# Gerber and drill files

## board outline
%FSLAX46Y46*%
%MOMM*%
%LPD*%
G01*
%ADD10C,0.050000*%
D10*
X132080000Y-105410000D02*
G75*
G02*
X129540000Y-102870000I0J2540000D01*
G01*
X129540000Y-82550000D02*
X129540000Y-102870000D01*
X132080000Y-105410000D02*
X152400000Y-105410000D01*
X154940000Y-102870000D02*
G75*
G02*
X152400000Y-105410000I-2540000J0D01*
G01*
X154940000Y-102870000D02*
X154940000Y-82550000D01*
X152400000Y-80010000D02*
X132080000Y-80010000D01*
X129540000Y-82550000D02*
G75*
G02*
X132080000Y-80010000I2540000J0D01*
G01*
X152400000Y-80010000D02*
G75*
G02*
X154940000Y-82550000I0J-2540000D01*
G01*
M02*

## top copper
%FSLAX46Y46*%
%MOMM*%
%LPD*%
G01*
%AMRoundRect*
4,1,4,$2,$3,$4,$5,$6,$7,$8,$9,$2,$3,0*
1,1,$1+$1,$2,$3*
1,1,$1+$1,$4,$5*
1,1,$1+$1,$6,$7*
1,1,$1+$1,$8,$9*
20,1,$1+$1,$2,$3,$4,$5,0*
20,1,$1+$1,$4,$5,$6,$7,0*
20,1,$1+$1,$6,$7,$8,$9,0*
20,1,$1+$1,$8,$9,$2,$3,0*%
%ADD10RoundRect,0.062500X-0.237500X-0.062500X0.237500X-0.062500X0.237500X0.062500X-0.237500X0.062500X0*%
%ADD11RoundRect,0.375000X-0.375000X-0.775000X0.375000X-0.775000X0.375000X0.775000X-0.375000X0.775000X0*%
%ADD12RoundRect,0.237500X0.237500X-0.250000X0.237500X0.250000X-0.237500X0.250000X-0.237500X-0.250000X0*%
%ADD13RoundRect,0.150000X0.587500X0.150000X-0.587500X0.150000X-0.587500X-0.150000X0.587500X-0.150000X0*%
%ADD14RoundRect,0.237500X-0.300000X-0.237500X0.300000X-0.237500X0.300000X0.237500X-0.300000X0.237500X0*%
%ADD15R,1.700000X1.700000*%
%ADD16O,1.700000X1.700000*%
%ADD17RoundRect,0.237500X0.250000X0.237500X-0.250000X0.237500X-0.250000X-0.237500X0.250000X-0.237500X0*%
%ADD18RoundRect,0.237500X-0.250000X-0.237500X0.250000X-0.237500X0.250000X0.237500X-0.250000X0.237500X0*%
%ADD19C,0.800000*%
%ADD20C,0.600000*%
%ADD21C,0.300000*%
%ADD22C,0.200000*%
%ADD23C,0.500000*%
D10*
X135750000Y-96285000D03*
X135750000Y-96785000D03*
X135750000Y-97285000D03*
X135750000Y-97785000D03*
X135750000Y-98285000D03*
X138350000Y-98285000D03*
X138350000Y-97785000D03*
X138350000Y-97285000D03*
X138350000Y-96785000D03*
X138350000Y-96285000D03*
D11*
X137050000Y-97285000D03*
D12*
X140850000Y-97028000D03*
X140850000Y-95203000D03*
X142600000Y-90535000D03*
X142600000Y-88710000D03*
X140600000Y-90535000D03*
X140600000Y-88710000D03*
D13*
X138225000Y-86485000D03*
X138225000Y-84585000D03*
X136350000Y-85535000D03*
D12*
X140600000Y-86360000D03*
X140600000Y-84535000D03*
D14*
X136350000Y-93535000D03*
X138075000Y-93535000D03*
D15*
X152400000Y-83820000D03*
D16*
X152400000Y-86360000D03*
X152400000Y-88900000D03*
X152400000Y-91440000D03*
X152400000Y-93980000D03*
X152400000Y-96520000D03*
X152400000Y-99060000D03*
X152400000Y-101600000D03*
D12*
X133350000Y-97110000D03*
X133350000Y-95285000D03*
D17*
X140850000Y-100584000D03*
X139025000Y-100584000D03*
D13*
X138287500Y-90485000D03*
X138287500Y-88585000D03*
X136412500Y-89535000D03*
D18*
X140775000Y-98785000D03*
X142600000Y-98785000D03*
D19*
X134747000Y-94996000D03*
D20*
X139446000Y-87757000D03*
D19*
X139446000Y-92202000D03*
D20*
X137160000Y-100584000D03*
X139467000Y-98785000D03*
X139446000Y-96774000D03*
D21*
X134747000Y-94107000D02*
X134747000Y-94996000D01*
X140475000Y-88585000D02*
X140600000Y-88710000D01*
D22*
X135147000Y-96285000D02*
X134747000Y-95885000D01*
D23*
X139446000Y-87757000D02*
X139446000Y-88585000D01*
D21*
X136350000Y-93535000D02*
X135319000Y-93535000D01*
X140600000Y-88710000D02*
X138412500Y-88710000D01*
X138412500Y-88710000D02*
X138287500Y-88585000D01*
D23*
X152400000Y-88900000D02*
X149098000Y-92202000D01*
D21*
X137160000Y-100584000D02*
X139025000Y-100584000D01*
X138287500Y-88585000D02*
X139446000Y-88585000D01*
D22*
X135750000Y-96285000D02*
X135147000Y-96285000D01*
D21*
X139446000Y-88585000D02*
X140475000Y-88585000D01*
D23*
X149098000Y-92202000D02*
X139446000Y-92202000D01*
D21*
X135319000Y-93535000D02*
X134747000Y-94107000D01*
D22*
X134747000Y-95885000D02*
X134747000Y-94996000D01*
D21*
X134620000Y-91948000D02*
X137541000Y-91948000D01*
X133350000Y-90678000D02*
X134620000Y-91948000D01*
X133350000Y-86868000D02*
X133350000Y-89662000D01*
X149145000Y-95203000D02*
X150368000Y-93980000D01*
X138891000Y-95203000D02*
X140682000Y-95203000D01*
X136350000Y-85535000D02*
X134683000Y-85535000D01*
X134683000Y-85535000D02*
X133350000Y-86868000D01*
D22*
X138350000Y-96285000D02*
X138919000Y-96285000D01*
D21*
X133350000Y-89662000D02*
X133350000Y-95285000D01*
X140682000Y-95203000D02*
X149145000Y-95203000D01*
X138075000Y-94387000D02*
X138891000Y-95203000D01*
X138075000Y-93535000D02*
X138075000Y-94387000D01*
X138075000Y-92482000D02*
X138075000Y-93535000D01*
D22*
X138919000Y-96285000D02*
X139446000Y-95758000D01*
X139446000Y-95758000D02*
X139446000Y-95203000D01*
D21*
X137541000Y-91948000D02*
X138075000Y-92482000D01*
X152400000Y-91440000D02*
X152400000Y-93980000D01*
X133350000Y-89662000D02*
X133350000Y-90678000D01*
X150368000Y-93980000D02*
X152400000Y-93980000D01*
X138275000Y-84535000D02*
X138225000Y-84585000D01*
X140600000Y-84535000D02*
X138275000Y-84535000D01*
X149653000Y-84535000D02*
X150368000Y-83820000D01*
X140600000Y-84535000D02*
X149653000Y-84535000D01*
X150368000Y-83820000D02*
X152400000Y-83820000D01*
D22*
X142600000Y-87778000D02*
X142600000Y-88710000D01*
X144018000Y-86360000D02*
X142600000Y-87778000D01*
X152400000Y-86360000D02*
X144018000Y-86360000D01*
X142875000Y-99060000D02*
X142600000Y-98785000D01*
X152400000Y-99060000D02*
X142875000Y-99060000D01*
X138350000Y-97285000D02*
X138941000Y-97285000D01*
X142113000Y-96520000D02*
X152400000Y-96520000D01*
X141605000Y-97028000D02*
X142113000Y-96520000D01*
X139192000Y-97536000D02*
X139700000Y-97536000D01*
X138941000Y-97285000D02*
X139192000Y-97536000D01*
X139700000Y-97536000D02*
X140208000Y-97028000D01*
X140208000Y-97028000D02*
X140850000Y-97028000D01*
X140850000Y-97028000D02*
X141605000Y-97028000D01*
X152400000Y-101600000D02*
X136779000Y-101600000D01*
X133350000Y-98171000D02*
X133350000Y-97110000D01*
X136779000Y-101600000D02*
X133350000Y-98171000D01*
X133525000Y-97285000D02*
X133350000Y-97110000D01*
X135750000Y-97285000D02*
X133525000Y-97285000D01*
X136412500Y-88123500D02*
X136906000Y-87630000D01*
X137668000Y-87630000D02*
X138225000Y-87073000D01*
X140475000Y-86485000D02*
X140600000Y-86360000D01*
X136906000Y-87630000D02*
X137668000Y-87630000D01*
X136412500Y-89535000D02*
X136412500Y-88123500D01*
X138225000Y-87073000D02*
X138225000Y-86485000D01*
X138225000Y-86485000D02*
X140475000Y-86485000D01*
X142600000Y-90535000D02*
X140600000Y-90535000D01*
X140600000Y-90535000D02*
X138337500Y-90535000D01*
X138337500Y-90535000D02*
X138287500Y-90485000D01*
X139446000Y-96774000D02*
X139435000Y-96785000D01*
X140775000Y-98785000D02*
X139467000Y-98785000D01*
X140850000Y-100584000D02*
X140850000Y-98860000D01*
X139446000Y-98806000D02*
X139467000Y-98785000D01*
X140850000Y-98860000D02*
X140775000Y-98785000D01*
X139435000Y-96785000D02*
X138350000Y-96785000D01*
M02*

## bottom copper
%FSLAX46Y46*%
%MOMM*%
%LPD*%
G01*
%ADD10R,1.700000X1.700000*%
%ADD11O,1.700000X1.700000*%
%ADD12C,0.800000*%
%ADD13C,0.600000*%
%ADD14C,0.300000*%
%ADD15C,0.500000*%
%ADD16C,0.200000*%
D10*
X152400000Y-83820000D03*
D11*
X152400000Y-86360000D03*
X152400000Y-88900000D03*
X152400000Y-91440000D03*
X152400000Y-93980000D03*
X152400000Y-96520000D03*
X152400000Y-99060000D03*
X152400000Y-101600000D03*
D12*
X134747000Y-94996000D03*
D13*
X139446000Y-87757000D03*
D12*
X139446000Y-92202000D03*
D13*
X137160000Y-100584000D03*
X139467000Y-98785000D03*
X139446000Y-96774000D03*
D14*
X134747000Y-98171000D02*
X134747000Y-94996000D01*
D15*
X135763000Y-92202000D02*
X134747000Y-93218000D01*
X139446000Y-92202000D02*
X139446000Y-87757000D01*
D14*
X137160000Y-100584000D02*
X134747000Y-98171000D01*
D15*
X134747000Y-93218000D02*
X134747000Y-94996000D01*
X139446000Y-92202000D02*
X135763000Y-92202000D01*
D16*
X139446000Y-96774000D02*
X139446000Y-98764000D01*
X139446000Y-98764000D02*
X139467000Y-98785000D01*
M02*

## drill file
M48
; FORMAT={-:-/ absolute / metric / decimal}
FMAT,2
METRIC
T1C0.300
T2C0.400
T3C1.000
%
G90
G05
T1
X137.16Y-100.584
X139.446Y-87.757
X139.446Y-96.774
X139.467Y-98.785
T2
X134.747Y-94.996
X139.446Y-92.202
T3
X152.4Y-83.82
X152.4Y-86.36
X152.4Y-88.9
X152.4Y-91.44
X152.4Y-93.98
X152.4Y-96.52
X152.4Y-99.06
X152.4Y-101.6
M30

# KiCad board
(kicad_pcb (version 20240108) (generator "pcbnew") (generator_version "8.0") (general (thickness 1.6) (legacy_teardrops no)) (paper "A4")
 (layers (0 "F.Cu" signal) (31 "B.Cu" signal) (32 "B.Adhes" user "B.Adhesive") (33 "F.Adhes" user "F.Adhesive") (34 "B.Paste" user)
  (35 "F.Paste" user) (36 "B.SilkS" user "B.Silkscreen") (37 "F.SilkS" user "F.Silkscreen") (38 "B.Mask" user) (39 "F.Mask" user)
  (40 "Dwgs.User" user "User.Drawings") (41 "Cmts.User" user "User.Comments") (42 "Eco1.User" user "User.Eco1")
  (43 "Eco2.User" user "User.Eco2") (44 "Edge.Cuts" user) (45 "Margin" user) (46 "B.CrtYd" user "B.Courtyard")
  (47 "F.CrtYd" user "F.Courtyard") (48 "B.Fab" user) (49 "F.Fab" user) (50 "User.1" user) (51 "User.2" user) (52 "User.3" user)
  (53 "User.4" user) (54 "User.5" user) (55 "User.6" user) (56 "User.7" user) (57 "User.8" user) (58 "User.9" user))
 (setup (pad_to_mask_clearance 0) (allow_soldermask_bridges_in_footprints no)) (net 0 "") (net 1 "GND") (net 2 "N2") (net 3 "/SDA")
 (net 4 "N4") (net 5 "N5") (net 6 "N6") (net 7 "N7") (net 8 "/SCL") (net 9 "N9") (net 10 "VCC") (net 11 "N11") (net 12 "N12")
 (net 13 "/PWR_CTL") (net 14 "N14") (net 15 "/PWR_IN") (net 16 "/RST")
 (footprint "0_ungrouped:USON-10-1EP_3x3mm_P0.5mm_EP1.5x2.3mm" (layer "F.Cu") (at 137.05 97.285)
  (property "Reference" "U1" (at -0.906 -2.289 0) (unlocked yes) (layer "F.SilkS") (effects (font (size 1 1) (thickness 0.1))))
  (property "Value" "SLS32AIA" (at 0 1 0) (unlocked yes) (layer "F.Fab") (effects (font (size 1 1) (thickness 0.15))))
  (pad "1" smd roundrect (at -1.3 -1) (size 0.6 0.25) (layers "F.Cu" "F.Paste" "F.Mask") (roundrect_rratio 0.25) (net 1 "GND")
   (thermal_bridge_angle 45))
  (pad "2" smd roundrect (at -1.3 -0.5) (size 0.6 0.25) (layers "F.Cu" "F.Paste" "F.Mask") (roundrect_rratio 0.25) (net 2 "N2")
   (thermal_bridge_angle 45))
  (pad "3" smd roundrect (at -1.3 0) (size 0.6 0.25) (layers "F.Cu" "F.Paste" "F.Mask") (roundrect_rratio 0.25) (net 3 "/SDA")
   (thermal_bridge_angle 45))
  (pad "4" smd roundrect (at -1.3 0.5) (size 0.6 0.25) (layers "F.Cu" "F.Paste" "F.Mask") (roundrect_rratio 0.25) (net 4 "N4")
   (thermal_bridge_angle 45))
  (pad "5" smd roundrect (at -1.3 1) (size 0.6 0.25) (layers "F.Cu" "F.Paste" "F.Mask") (roundrect_rratio 0.25) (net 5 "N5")
   (thermal_bridge_angle 45))
  (pad "6" smd roundrect (at 1.3 1) (size 0.6 0.25) (layers "F.Cu" "F.Paste" "F.Mask") (roundrect_rratio 0.25) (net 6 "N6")
   (thermal_bridge_angle 45))
  (pad "7" smd roundrect (at 1.3 0.5) (size 0.6 0.25) (layers "F.Cu" "F.Paste" "F.Mask") (roundrect_rratio 0.25) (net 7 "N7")
   (thermal_bridge_angle 45))
  (pad "8" smd roundrect (at 1.3 0) (size 0.6 0.25) (layers "F.Cu" "F.Paste" "F.Mask") (roundrect_rratio 0.25) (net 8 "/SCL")
   (thermal_bridge_angle 45))
  (pad "9" smd roundrect (at 1.3 -0.5) (size 0.6 0.25) (layers "F.Cu" "F.Paste" "F.Mask") (roundrect_rratio 0.25) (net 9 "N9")
   (thermal_bridge_angle 45))
  (pad "10" smd roundrect (at 1.3 -1) (size 0.6 0.25) (layers "F.Cu" "F.Paste" "F.Mask") (roundrect_rratio 0.25) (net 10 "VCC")
   (thermal_bridge_angle 45))
  (pad "11" smd roundrect (at 0 0) (size 1.5 2.3) (layers "F.Cu" "F.Paste" "F.Mask") (roundrect_rratio 0.25) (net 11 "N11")
   (thermal_bridge_angle 45)))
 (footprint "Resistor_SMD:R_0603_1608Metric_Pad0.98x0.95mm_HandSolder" (layer "F.Cu") (at 140.85 96.1155 90)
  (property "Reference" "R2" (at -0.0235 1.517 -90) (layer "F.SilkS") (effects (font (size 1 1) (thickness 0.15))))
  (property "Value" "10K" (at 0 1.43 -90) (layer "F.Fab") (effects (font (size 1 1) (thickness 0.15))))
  (pad "1" smd roundrect (at -0.9125 0 90) (size 0.975 0.95) (layers "F.Cu" "F.Paste" "F.Mask") (roundrect_rratio 0.25) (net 8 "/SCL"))
  (pad "2" smd roundrect (at 0.9125 0 90) (size 0.975 0.95) (layers "F.Cu" "F.Paste" "F.Mask") (roundrect_rratio 0.25) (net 10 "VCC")))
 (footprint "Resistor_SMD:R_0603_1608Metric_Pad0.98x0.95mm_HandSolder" (layer "F.Cu") (at 142.6 89.6225 90)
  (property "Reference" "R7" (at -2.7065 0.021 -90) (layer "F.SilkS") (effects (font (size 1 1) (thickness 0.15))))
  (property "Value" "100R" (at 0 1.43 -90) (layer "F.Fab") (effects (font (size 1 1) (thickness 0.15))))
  (pad "1" smd roundrect (at -0.9125 0 90) (size 0.975 0.95) (layers "F.Cu" "F.Paste" "F.Mask") (roundrect_rratio 0.25) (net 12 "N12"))
  (pad "2" smd roundrect (at 0.9125 0 90) (size 0.975 0.95) (layers "F.Cu" "F.Paste" "F.Mask") (roundrect_rratio 0.25) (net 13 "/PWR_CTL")))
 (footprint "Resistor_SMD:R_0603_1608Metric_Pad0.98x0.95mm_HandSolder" (layer "F.Cu") (at 140.6 89.6225 90)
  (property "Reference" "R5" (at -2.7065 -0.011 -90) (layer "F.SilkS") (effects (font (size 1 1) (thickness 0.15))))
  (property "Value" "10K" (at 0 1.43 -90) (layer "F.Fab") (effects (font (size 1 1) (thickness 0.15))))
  (pad "1" smd roundrect (at -0.9125 0 90) (size 0.975 0.95) (layers "F.Cu" "F.Paste" "F.Mask") (roundrect_rratio 0.25) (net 12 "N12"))
  (pad "2" smd roundrect (at 0.9125 0 90) (size 0.975 0.95) (layers "F.Cu" "F.Paste" "F.Mask") (roundrect_rratio 0.25) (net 1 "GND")))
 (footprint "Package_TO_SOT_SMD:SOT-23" (layer "F.Cu") (at 137.2875 85.535 180)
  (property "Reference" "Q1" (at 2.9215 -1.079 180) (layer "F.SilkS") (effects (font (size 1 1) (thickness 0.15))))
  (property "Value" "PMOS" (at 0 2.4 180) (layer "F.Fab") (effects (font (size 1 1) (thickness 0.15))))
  (pad "1" smd roundrect (at -0.9375 -0.95 180) (size 1.475 0.6) (layers "F.Cu" "F.Paste" "F.Mask") (roundrect_rratio 0.25) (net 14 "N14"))
  (pad "2" smd roundrect (at -0.9375 0.95 180) (size 1.475 0.6) (layers "F.Cu" "F.Paste" "F.Mask") (roundrect_rratio 0.25)
   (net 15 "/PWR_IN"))
  (pad "3" smd roundrect (at 0.9375 0 180) (size 1.475 0.6) (layers "F.Cu" "F.Paste" "F.Mask") (roundrect_rratio 0.25) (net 10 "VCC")))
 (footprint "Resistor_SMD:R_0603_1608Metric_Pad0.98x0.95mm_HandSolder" (layer "F.Cu") (at 140.6 85.4475 90)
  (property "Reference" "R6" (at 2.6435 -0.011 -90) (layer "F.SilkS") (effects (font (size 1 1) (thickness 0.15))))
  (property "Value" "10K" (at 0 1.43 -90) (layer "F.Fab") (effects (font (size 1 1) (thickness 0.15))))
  (pad "1" smd roundrect (at -0.9125 0 90) (size 0.975 0.95) (layers "F.Cu" "F.Paste" "F.Mask") (roundrect_rratio 0.25) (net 14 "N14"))
  (pad "2" smd roundrect (at 0.9125 0 90) (size 0.975 0.95) (layers "F.Cu" "F.Paste" "F.Mask") (roundrect_rratio 0.25) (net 15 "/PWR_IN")))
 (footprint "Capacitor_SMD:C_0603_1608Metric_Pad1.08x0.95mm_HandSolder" (layer "F.Cu") (at 137.2125 93.535)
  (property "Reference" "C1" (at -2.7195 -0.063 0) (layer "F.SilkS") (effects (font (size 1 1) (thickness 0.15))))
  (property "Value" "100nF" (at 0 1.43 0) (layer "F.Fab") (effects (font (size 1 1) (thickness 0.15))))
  (pad "1" smd roundrect (at -0.8625 0) (size 1.075 0.95) (layers "F.Cu" "F.Paste" "F.Mask") (roundrect_rratio 0.25) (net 1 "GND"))
  (pad "2" smd roundrect (at 0.8625 0) (size 1.075 0.95) (layers "F.Cu" "F.Paste" "F.Mask") (roundrect_rratio 0.25) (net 10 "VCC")))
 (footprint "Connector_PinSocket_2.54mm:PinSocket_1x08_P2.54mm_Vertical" (layer "F.Cu") (at 152.4 83.82)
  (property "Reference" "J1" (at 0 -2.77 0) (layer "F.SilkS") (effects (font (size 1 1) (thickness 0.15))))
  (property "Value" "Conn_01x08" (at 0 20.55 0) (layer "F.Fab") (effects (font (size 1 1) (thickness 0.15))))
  (pad "1" thru_hole rect (at 0 0) (size 1.7 1.7) (drill 1) (layers "*.Cu" "*.Mask") (remove_unused_layers no) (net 15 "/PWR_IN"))
  (pad "2" thru_hole oval (at 0 2.54) (size 1.7 1.7) (drill 1) (layers "*.Cu" "*.Mask") (remove_unused_layers no) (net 13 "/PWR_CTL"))
  (pad "3" thru_hole oval (at 0 5.08) (size 1.7 1.7) (drill 1) (layers "*.Cu" "*.Mask") (remove_unused_layers no) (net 1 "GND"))
  (pad "4" thru_hole oval (at 0 7.62) (size 1.7 1.7) (drill 1) (layers "*.Cu" "*.Mask") (remove_unused_layers no) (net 10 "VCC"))
  (pad "5" thru_hole oval (at 0 10.16) (size 1.7 1.7) (drill 1) (layers "*.Cu" "*.Mask") (remove_unused_layers no) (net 10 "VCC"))
  (pad "6" thru_hole oval (at 0 12.7) (size 1.7 1.7) (drill 1) (layers "*.Cu" "*.Mask") (remove_unused_layers no) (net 8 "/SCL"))
  (pad "7" thru_hole oval (at 0 15.24) (size 1.7 1.7) (drill 1) (layers "*.Cu" "*.Mask") (remove_unused_layers no) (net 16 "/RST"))
  (pad "8" thru_hole oval (at 0 17.78) (size 1.7 1.7) (drill 1) (layers "*.Cu" "*.Mask") (remove_unused_layers no) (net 3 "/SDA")))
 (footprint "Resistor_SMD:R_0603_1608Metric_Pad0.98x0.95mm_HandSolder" (layer "F.Cu") (at 133.35 96.1975 90)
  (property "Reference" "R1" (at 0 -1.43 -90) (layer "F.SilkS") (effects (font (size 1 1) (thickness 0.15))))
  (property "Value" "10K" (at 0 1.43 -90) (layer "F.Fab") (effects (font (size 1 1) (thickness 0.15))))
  (pad "1" smd roundrect (at -0.9125 0 90) (size 0.975 0.95) (layers "F.Cu" "F.Paste" "F.Mask") (roundrect_rratio 0.25) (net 3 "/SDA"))
  (pad "2" smd roundrect (at 0.9125 0 90) (size 0.975 0.95) (layers "F.Cu" "F.Paste" "F.Mask") (roundrect_rratio 0.25) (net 10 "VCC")))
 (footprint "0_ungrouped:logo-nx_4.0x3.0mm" (layer "F.Cu") (at 133.223 102.489)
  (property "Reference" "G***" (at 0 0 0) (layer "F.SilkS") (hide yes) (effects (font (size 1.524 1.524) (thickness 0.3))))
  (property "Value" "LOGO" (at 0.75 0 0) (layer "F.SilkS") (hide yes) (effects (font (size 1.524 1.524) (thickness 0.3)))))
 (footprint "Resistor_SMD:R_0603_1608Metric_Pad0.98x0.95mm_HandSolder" (layer "F.Cu") (at 139.9375 100.584 180)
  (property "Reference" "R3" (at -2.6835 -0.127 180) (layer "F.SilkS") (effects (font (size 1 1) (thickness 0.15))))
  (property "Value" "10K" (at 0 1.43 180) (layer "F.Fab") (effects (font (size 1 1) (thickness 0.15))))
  (pad "1" smd roundrect (at -0.9125 0 180) (size 0.975 0.95) (layers "F.Cu" "F.Paste" "F.Mask") (roundrect_rratio 0.25) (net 9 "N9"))
  (pad "2" smd roundrect (at 0.9125 0 180) (size 0.975 0.95) (layers "F.Cu" "F.Paste" "F.Mask") (roundrect_rratio 0.25) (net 1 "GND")))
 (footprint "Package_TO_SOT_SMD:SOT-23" (layer "F.Cu") (at 137.35 89.535 180)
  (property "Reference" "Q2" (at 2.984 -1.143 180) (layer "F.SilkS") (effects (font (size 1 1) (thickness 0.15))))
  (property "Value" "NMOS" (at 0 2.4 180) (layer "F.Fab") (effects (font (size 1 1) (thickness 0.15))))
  (pad "1" smd roundrect (at -0.9375 -0.95 180) (size 1.475 0.6) (layers "F.Cu" "F.Paste" "F.Mask") (roundrect_rratio 0.25) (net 12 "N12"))
  (pad "2" smd roundrect (at -0.9375 0.95 180) (size 1.475 0.6) (layers "F.Cu" "F.Paste" "F.Mask") (roundrect_rratio 0.25) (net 1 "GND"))
  (pad "3" smd roundrect (at 0.9375 0 180) (size 1.475 0.6) (layers "F.Cu" "F.Paste" "F.Mask") (roundrect_rratio 0.25) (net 14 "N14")))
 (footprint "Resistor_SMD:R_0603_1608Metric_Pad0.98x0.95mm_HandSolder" (layer "F.Cu") (at 141.6875 98.785)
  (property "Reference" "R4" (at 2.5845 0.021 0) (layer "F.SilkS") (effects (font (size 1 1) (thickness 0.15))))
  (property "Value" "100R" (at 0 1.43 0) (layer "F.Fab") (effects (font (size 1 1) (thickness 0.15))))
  (pad "1" smd roundrect (at -0.9125 0) (size 0.975 0.95) (layers "F.Cu" "F.Paste" "F.Mask") (roundrect_rratio 0.25) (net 9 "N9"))
  (pad "2" smd roundrect (at 0.9125 0) (size 0.975 0.95) (layers "F.Cu" "F.Paste" "F.Mask") (roundrect_rratio 0.25) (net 16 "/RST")))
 (gr_arc (start 132.08 105.41) (mid 130.283949 104.666051) (end 129.54 102.87) (stroke (width 0.05) (type default)) (layer "Edge.Cuts"))
 (gr_line (start 129.54 82.55) (end 129.54 102.87) (stroke (width 0.05) (type default)) (layer "Edge.Cuts"))
 (gr_line (start 132.08 105.41) (end 152.4 105.41) (stroke (width 0.05) (type default)) (layer "Edge.Cuts"))
 (gr_arc (start 154.94 102.87) (mid 154.196051 104.666051) (end 152.4 105.41) (stroke (width 0.05) (type default)) (layer "Edge.Cuts"))
 (gr_line (start 154.94 102.87) (end 154.94 82.55) (stroke (width 0.05) (type default)) (layer "Edge.Cuts"))
 (gr_line (start 152.4 80.01) (end 132.08 80.01) (stroke (width 0.05) (type default)) (layer "Edge.Cuts"))
 (gr_arc (start 129.54 82.55) (mid 130.283949 80.753949) (end 132.08 80.01) (stroke (width 0.05) (type default)) (layer "Edge.Cuts"))
 (gr_arc (start 152.4 80.01) (mid 154.196051 80.753949) (end 154.94 82.55) (stroke (width 0.05) (type default)) (layer "Edge.Cuts"))
 (segment (start 134.747 94.107) (end 134.747 94.996) (width 0.3) (layer "F.Cu") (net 1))
 (segment (start 140.475 88.585) (end 140.6 88.71) (width 0.3) (layer "F.Cu") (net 1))
 (segment (start 135.147 96.285) (end 134.747 95.885) (width 0.2) (layer "F.Cu") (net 1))
 (segment (start 139.446 87.757) (end 139.446 88.585) (width 0.5) (layer "F.Cu") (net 1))
 (segment (start 136.35 93.535) (end 135.319 93.535) (width 0.3) (layer "F.Cu") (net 1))
 (segment (start 140.6 88.71) (end 138.4125 88.71) (width 0.3) (layer "F.Cu") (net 1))
 (segment (start 138.4125 88.71) (end 138.2875 88.585) (width 0.3) (layer "F.Cu") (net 1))
 (segment (start 152.4 88.9) (end 149.098 92.202) (width 0.5) (layer "F.Cu") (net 1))
 (segment (start 137.16 100.584) (end 139.025 100.584) (width 0.3) (layer "F.Cu") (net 1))
 (segment (start 138.2875 88.585) (end 139.446 88.585) (width 0.3) (layer "F.Cu") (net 1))
 (segment (start 135.75 96.285) (end 135.147 96.285) (width 0.2) (layer "F.Cu") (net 1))
 (segment (start 139.446 88.585) (end 140.475 88.585) (width 0.3) (layer "F.Cu") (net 1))
 (segment (start 149.098 92.202) (end 139.446 92.202) (width 0.5) (layer "F.Cu") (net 1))
 (segment (start 135.319 93.535) (end 134.747 94.107) (width 0.3) (layer "F.Cu") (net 1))
 (segment (start 134.747 95.885) (end 134.747 94.996) (width 0.2) (layer "F.Cu") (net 1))
 (via (at 134.747 94.996) (size 0.8) (drill 0.4) (layers "F.Cu" "B.Cu") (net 1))
 (via (at 139.446 87.757) (size 0.6) (drill 0.3) (layers "F.Cu" "B.Cu") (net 1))
 (via (at 139.446 92.202) (size 0.8) (drill 0.4) (layers "F.Cu" "B.Cu") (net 1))
 (via (at 137.16 100.584) (size 0.6) (drill 0.3) (layers "F.Cu" "B.Cu") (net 1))
 (segment (start 134.747 98.171) (end 134.747 94.996) (width 0.3) (layer "B.Cu") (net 1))
 (segment (start 135.763 92.202) (end 134.747 93.218) (width 0.5) (layer "B.Cu") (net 1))
 (segment (start 139.446 92.202) (end 139.446 87.757) (width 0.5) (layer "B.Cu") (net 1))
 (segment (start 137.16 100.584) (end 134.747 98.171) (width 0.3) (layer "B.Cu") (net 1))
 (segment (start 134.747 93.218) (end 134.747 94.996) (width 0.5) (layer "B.Cu") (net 1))
 (segment (start 139.446 92.202) (end 135.763 92.202) (width 0.5) (layer "B.Cu") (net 1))
 (segment (start 134.62 91.948) (end 137.541 91.948) (width 0.3) (layer "F.Cu") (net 10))
 (segment (start 133.35 90.678) (end 134.62 91.948) (width 0.3) (layer "F.Cu") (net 10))
 (segment (start 133.35 86.868) (end 133.35 89.662) (width 0.3) (layer "F.Cu") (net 10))
 (segment (start 149.145 95.203) (end 150.368 93.98) (width 0.3) (layer "F.Cu") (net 10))
 (segment (start 138.891 95.203) (end 140.682 95.203) (width 0.3) (layer "F.Cu") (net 10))
 (segment (start 136.35 85.535) (end 134.683 85.535) (width 0.3) (layer "F.Cu") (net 10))
 (segment (start 134.683 85.535) (end 133.35 86.868) (width 0.3) (layer "F.Cu") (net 10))
 (segment (start 138.35 96.285) (end 138.919 96.285) (width 0.2) (layer "F.Cu") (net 10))
 (segment (start 133.35 89.662) (end 133.35 95.285) (width 0.3) (layer "F.Cu") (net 10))
 (segment (start 140.682 95.203) (end 149.145 95.203) (width 0.3) (layer "F.Cu") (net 10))
 (segment (start 138.075 94.387) (end 138.891 95.203) (width 0.3) (layer "F.Cu") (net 10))
 (segment (start 138.075 93.535) (end 138.075 94.387) (width 0.3) (layer "F.Cu") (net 10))
 (segment (start 138.075 92.482) (end 138.075 93.535) (width 0.3) (layer "F.Cu") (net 10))
 (segment (start 138.919 96.285) (end 139.446 95.758) (width 0.2) (layer "F.Cu") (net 10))
 (segment (start 139.446 95.758) (end 139.446 95.203) (width 0.2) (layer "F.Cu") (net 10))
 (segment (start 137.541 91.948) (end 138.075 92.482) (width 0.3) (layer "F.Cu") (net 10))
 (segment (start 152.4 91.44) (end 152.4 93.98) (width 0.3) (layer "F.Cu") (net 10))
 (segment (start 133.35 89.662) (end 133.35 90.678) (width 0.3) (layer "F.Cu") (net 10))
 (segment (start 150.368 93.98) (end 152.4 93.98) (width 0.3) (layer "F.Cu") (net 10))
 (segment (start 138.275 84.535) (end 138.225 84.585) (width 0.3) (layer "F.Cu") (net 15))
 (segment (start 140.6 84.535) (end 138.275 84.535) (width 0.3) (layer "F.Cu") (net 15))
 (segment (start 149.653 84.535) (end 150.368 83.82) (width 0.3) (layer "F.Cu") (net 15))
 (segment (start 140.6 84.535) (end 149.653 84.535) (width 0.3) (layer "F.Cu") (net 15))
 (segment (start 150.368 83.82) (end 152.4 83.82) (width 0.3) (layer "F.Cu") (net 15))
 (segment (start 142.6 87.778) (end 142.6 88.71) (width 0.2) (layer "F.Cu") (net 13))
 (segment (start 144.018 86.36) (end 142.6 87.778) (width 0.2) (layer "F.Cu") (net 13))
 (segment (start 152.4 86.36) (end 144.018 86.36) (width 0.2) (layer "F.Cu") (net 13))
 (segment (start 142.875 99.06) (end 142.6 98.785) (width 0.2) (layer "F.Cu") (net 16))
 (segment (start 152.4 99.06) (end 142.875 99.06) (width 0.2) (layer "F.Cu") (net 16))
 (segment (start 138.35 97.285) (end 138.941 97.285) (width 0.2) (layer "F.Cu") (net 8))
 (segment (start 142.113 96.52) (end 152.4 96.52) (width 0.2) (layer "F.Cu") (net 8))
 (segment (start 141.605 97.028) (end 142.113 96.52) (width 0.2) (layer "F.Cu") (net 8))
 (segment (start 139.192 97.536) (end 139.7 97.536) (width 0.2) (layer "F.Cu") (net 8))
 (segment (start 138.941 97.285) (end 139.192 97.536) (width 0.2) (layer "F.Cu") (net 8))
 (segment (start 139.7 97.536) (end 140.208 97.028) (width 0.2) (layer "F.Cu") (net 8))
 (segment (start 140.208 97.028) (end 140.85 97.028) (width 0.2) (layer "F.Cu") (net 8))
 (segment (start 140.85 97.028) (end 141.605 97.028) (width 0.2) (layer "F.Cu") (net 8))
 (segment (start 152.4 101.6) (end 136.779 101.6) (width 0.2) (layer "F.Cu") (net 3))
 (segment (start 133.35 98.171) (end 133.35 97.11) (width 0.2) (layer "F.Cu") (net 3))
 (segment (start 136.779 101.6) (end 133.35 98.171) (width 0.2) (layer "F.Cu") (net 3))
 (segment (start 133.525 97.285) (end 133.35 97.11) (width 0.2) (layer "F.Cu") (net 3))
 (segment (start 135.75 97.285) (end 133.525 97.285) (width 0.2) (layer "F.Cu") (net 3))
 (segment (start 136.4125 88.1235) (end 136.906 87.63) (width 0.2) (layer "F.Cu") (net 14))
 (segment (start 137.668 87.63) (end 138.225 87.073) (width 0.2) (layer "F.Cu") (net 14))
 (segment (start 140.475 86.485) (end 140.6 86.36) (width 0.2) (layer "F.Cu") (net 14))
 (segment (start 136.906 87.63) (end 137.668 87.63) (width 0.2) (layer "F.Cu") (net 14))
 (segment (start 136.4125 89.535) (end 136.4125 88.1235) (width 0.2) (layer "F.Cu") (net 14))
 (segment (start 138.225 87.073) (end 138.225 86.485) (width 0.2) (layer "F.Cu") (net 14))
 (segment (start 138.225 86.485) (end 140.475 86.485) (width 0.2) (layer "F.Cu") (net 14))
 (segment (start 142.6 90.535) (end 140.6 90.535) (width 0.2) (layer "F.Cu") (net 12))
 (segment (start 140.6 90.535) (end 138.3375 90.535) (width 0.2) (layer "F.Cu") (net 12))
 (segment (start 138.3375 90.535) (end 138.2875 90.485) (width 0.2) (layer "F.Cu") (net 12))
 (segment (start 139.446 96.774) (end 139.435 96.785) (width 0.2) (layer "F.Cu") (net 9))
 (segment (start 140.775 98.785) (end 139.467 98.785) (width 0.2) (layer "F.Cu") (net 9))
 (segment (start 140.85 100.584) (end 140.85 98.86) (width 0.2) (layer "F.Cu") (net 9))
 (segment (start 139.446 98.806) (end 139.467 98.785) (width 0.2) (layer "F.Cu") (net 9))
 (segment (start 140.85 98.86) (end 140.775 98.785) (width 0.2) (layer "F.Cu") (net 9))
 (segment (start 139.435 96.785) (end 138.35 96.785) (width 0.2) (layer "F.Cu") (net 9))
 (via (at 139.467 98.785) (size 0.6) (drill 0.3) (layers "F.Cu" "B.Cu") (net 9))
 (via (at 139.446 96.774) (size 0.6) (drill 0.3) (layers "F.Cu" "B.Cu") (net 9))
 (segment (start 139.446 96.774) (end 139.446 98.764) (width 0.2) (layer "B.Cu") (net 9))
 (segment (start 139.446 98.764) (end 139.467 98.785) (width 0.2) (layer "B.Cu") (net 9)))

